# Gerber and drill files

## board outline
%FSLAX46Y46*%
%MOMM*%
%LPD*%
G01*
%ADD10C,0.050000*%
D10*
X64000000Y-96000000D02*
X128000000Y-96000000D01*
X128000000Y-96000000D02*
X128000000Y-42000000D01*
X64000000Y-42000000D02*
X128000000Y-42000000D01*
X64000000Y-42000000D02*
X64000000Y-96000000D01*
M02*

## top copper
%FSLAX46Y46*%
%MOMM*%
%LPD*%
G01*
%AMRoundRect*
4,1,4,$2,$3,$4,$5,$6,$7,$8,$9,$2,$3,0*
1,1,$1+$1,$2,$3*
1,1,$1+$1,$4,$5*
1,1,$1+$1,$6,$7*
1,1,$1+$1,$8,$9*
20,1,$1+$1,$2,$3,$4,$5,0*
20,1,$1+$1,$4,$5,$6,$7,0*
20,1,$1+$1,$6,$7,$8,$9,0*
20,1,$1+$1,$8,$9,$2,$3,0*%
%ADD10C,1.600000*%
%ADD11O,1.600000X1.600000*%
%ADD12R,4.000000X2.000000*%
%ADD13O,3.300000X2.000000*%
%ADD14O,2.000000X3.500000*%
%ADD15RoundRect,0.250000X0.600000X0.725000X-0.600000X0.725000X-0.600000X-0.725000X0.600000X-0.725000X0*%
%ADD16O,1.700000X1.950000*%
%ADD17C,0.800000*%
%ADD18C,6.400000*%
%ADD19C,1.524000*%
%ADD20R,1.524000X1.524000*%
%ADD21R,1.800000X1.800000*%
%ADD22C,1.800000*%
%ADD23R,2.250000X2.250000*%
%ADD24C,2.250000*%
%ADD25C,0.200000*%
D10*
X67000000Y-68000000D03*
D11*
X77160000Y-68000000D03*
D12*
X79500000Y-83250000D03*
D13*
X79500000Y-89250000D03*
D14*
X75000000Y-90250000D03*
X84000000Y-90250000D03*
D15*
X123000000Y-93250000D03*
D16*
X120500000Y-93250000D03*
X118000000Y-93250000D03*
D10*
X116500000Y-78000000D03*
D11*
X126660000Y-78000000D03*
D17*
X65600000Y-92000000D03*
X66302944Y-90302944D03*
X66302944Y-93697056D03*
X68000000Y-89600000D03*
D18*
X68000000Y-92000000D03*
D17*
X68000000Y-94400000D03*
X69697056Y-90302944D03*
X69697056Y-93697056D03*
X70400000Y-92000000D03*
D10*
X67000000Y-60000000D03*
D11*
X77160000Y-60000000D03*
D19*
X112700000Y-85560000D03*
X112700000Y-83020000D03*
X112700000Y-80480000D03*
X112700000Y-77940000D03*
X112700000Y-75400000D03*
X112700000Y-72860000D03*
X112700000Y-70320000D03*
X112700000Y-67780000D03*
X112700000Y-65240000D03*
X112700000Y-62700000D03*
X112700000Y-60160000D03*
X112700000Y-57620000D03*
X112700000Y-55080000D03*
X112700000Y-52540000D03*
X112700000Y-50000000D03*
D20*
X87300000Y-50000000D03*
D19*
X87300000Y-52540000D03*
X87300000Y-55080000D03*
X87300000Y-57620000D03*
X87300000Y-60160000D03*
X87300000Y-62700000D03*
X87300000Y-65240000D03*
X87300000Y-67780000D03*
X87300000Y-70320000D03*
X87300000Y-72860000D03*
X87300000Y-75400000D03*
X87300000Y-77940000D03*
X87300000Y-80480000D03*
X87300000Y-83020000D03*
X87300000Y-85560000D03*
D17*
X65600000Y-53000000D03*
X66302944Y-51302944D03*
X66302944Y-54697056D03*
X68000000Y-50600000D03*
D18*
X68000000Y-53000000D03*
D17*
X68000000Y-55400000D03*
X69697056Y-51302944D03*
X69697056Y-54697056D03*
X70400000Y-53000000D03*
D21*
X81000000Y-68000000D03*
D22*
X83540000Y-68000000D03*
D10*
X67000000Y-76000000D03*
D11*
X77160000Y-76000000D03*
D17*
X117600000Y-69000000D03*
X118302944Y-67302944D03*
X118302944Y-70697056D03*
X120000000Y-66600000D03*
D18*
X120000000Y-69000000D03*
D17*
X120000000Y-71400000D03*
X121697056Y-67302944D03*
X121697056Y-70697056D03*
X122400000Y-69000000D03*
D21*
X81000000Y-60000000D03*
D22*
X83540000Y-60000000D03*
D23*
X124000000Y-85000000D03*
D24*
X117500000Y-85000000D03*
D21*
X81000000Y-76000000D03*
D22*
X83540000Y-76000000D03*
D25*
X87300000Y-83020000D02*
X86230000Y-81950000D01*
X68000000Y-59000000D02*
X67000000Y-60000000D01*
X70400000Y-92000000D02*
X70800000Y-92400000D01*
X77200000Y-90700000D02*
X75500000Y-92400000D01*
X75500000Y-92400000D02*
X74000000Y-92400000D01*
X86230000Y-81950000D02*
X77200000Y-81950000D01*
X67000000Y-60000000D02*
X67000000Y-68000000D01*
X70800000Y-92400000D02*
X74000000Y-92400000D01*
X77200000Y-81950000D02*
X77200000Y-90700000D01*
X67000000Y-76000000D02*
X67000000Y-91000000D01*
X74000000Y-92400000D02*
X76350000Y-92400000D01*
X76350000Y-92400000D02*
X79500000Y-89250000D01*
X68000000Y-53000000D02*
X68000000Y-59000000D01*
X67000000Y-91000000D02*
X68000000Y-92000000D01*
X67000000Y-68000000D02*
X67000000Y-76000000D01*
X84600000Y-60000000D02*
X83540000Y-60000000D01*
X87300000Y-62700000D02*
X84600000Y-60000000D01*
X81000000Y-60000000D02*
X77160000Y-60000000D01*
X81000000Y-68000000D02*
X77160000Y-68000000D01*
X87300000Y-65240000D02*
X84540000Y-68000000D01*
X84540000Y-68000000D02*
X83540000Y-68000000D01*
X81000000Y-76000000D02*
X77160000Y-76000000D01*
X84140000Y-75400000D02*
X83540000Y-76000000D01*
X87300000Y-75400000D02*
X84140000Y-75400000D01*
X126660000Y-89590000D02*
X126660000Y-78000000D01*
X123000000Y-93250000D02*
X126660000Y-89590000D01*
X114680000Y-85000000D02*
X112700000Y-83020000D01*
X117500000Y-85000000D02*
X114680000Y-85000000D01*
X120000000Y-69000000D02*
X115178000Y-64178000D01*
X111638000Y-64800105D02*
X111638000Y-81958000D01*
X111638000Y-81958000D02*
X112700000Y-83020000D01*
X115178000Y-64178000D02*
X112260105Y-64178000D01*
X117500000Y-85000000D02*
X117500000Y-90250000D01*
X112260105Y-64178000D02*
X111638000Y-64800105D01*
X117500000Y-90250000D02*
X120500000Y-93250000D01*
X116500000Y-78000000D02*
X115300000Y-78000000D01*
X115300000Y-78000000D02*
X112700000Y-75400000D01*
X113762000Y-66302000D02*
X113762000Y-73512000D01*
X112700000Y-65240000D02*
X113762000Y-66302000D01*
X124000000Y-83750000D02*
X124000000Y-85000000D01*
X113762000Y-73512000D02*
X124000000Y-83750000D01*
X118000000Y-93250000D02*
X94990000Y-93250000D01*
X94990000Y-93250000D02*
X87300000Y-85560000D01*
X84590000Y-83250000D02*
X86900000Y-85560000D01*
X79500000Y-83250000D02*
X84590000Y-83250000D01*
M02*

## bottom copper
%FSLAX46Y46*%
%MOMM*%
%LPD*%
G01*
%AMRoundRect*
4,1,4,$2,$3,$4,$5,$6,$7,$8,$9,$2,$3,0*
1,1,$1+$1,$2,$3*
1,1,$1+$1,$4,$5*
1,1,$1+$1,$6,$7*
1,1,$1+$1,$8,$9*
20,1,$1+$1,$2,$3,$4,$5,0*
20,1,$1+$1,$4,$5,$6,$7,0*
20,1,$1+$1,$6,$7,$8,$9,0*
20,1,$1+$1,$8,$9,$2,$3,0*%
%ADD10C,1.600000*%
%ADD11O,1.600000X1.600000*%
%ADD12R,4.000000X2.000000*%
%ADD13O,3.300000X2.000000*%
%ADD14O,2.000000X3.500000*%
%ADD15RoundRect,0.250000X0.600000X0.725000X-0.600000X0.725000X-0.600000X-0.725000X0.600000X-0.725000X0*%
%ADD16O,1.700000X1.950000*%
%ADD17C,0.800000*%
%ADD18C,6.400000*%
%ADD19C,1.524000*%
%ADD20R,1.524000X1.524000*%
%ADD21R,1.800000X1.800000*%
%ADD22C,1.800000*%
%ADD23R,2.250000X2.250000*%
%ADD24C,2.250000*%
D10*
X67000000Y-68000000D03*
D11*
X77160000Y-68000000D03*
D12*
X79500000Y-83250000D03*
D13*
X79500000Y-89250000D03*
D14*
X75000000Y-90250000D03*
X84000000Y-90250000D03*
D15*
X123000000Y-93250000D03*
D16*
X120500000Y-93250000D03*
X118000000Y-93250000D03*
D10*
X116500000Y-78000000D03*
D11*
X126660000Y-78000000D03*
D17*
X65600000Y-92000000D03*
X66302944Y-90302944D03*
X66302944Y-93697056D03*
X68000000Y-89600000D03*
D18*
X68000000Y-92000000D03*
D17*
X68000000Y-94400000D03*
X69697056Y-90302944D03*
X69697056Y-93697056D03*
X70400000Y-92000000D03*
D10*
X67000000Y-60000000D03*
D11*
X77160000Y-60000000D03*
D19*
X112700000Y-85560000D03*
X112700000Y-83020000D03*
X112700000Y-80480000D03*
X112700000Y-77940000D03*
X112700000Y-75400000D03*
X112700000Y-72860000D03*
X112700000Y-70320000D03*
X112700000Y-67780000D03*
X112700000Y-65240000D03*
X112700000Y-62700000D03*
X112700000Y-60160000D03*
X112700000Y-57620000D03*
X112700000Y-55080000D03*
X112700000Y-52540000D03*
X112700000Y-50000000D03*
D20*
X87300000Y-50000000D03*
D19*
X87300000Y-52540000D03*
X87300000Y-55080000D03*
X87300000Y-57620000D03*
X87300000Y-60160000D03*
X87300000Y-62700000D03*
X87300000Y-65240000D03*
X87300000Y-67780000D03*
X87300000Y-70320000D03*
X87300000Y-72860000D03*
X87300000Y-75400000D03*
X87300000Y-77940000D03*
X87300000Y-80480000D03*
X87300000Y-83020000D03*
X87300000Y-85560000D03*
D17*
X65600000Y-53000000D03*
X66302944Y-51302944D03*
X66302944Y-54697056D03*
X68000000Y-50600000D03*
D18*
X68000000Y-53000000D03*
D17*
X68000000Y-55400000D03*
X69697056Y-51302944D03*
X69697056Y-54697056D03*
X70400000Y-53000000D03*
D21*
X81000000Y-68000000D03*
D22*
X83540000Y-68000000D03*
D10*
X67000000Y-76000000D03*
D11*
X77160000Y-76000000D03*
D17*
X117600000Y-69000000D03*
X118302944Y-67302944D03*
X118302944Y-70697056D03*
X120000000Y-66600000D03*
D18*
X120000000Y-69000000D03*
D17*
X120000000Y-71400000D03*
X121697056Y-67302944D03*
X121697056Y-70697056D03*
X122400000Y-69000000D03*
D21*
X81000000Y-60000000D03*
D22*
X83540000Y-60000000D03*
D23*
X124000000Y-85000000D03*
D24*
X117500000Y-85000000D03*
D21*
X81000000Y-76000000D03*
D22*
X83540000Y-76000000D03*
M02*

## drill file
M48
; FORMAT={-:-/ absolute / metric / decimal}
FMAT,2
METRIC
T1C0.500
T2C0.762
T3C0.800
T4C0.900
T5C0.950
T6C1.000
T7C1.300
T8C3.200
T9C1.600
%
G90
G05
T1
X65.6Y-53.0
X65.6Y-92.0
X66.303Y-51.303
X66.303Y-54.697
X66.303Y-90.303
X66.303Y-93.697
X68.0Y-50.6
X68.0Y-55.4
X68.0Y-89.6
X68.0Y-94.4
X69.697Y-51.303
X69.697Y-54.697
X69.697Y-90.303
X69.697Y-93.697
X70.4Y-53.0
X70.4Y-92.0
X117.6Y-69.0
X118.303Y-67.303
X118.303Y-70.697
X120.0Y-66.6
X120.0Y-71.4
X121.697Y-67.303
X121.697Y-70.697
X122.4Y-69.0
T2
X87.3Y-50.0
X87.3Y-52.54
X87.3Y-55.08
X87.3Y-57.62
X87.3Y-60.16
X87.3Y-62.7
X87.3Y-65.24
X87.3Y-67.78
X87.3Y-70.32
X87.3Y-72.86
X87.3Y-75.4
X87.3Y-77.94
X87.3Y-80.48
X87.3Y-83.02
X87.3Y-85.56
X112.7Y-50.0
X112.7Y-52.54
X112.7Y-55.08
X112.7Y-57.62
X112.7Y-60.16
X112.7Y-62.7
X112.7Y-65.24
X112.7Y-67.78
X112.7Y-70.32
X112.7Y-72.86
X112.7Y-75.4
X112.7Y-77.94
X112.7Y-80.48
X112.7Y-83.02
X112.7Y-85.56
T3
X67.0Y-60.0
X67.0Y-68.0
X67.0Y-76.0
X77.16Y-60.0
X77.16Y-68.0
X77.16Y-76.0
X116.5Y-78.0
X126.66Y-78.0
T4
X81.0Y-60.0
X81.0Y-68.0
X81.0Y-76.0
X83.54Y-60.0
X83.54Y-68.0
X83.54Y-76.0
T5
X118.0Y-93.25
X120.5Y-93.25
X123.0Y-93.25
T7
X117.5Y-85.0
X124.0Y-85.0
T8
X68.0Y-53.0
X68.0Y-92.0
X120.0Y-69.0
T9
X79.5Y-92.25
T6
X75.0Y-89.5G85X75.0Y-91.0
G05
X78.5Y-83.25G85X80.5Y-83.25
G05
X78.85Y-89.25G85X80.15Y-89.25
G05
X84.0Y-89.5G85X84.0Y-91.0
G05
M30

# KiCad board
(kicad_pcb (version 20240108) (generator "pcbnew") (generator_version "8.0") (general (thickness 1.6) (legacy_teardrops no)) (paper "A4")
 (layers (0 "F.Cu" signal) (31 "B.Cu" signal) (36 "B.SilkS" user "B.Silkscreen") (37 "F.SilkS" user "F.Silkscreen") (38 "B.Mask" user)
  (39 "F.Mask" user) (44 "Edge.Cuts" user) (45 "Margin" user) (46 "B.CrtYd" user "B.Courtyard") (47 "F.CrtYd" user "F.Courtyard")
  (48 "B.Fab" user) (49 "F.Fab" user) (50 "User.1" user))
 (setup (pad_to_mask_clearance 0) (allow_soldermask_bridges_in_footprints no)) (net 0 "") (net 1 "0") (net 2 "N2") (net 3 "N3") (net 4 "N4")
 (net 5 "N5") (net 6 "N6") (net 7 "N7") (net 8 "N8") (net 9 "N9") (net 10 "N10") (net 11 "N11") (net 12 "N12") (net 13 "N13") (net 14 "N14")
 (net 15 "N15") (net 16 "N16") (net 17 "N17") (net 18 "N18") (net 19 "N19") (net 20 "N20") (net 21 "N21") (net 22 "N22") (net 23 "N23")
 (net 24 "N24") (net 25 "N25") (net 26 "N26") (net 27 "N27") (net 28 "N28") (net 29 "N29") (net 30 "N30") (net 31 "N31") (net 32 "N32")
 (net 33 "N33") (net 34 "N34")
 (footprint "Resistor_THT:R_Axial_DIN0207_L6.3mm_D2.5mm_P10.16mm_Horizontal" (layer "F.Cu") (at 67 68)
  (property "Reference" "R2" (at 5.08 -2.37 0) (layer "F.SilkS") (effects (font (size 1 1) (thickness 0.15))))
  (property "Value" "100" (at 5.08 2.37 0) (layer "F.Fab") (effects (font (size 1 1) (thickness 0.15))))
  (pad "1" thru_hole circle (at 0 0) (size 1.6 1.6) (drill 0.8) (layers "*.Cu" "*.Mask") (remove_unused_layers no) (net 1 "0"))
  (pad "2" thru_hole oval (at 10.16 0) (size 1.6 1.6) (drill 0.8) (layers "*.Cu" "*.Mask") (remove_unused_layers no) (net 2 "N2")))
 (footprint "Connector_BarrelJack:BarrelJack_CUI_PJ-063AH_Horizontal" (layer "F.Cu") (at 79.5 83.25)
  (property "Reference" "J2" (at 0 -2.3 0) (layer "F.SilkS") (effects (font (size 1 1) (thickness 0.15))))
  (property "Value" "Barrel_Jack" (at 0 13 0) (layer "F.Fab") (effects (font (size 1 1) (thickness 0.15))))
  (pad "" np_thru_hole circle (at 0 9) (size 1.6 1.6) (drill 1.6) (layers "*.Cu" "*.Mask"))
  (pad "1" thru_hole rect (at 0 0) (size 4 2) (drill oval 3 1) (layers "*.Cu" "*.Mask") (remove_unused_layers no) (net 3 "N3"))
  (pad "2" thru_hole oval (at 0 6) (size 3.3 2) (drill oval 2.3 1) (layers "*.Cu" "*.Mask") (remove_unused_layers no) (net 1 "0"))
  (pad "MP" thru_hole oval (at -4.5 7) (size 2 3.5) (drill oval 1 2.5) (layers "*.Cu" "*.Mask") (remove_unused_layers no))
  (pad "MP" thru_hole oval (at 4.5 7) (size 2 3.5) (drill oval 1 2.5) (layers "*.Cu" "*.Mask") (remove_unused_layers no)))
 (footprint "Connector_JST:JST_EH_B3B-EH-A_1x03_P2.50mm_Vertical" (layer "F.Cu") (at 123 93.25 180)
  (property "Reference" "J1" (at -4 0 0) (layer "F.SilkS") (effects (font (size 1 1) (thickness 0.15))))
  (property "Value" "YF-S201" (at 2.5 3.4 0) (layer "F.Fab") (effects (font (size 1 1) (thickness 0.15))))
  (pad "1" thru_hole roundrect (at 0 0 180) (size 1.7 1.95) (drill 0.95) (layers "*.Cu" "*.Mask") (remove_unused_layers no)
   (roundrect_rratio 0.147059) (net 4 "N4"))
  (pad "2" thru_hole oval (at 2.5 0 180) (size 1.7 1.95) (drill 0.95) (layers "*.Cu" "*.Mask") (remove_unused_layers no) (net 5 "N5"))
  (pad "3" thru_hole oval (at 5 0 180) (size 1.7 1.95) (drill 0.95) (layers "*.Cu" "*.Mask") (remove_unused_layers no) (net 3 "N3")))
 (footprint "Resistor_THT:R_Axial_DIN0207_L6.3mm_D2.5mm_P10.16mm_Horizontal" (layer "F.Cu") (at 116.5 78)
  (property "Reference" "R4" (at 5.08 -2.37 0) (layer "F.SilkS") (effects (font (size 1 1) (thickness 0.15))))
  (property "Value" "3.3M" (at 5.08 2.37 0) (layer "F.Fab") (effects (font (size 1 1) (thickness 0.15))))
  (pad "1" thru_hole circle (at 0 0) (size 1.6 1.6) (drill 0.8) (layers "*.Cu" "*.Mask") (remove_unused_layers no) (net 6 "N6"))
  (pad "2" thru_hole oval (at 10.16 0) (size 1.6 1.6) (drill 0.8) (layers "*.Cu" "*.Mask") (remove_unused_layers no) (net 4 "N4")))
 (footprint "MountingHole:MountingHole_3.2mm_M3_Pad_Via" (layer "F.Cu") (at 68 92)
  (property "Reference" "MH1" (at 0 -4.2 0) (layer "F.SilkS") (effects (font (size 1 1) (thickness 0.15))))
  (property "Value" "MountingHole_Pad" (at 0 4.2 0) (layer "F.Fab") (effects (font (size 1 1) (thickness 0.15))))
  (pad "1" thru_hole circle (at -2.4 0) (size 0.8 0.8) (drill 0.5) (layers "*.Cu" "*.Mask") (remove_unused_layers no) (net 1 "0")
   (zone_connect 2))
  (pad "1" thru_hole circle (at -1.697056 -1.697056) (size 0.8 0.8) (drill 0.5) (layers "*.Cu" "*.Mask") (remove_unused_layers no)
   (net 1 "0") (zone_connect 2))
  (pad "1" thru_hole circle (at -1.697056 1.697056) (size 0.8 0.8) (drill 0.5) (layers "*.Cu" "*.Mask") (remove_unused_layers no)
   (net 1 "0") (zone_connect 2))
  (pad "1" thru_hole circle (at 0 -2.4) (size 0.8 0.8) (drill 0.5) (layers "*.Cu" "*.Mask") (remove_unused_layers no) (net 1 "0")
   (zone_connect 2))
  (pad "1" thru_hole circle (at 0 0) (size 6.4 6.4) (drill 3.2) (layers "*.Cu" "*.Mask") (remove_unused_layers no) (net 1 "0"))
  (pad "1" thru_hole circle (at 0 2.4) (size 0.8 0.8) (drill 0.5) (layers "*.Cu" "*.Mask") (remove_unused_layers no) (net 1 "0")
   (zone_connect 2))
  (pad "1" thru_hole circle (at 1.697056 -1.697056) (size 0.8 0.8) (drill 0.5) (layers "*.Cu" "*.Mask") (remove_unused_layers no)
   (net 1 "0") (zone_connect 2))
  (pad "1" thru_hole circle (at 1.697056 1.697056) (size 0.8 0.8) (drill 0.5) (layers "*.Cu" "*.Mask") (remove_unused_layers no) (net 1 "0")
   (zone_connect 2))
  (pad "1" thru_hole circle (at 2.4 0) (size 0.8 0.8) (drill 0.5) (layers "*.Cu" "*.Mask") (remove_unused_layers no) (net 1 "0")
   (zone_connect 2)))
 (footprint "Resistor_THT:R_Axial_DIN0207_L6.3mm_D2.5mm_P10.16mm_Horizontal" (layer "F.Cu") (at 67 60)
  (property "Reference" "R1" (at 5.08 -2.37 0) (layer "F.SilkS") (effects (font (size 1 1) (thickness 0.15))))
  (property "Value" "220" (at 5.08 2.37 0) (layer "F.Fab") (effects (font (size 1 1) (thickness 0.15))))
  (pad "1" thru_hole circle (at 0 0) (size 1.6 1.6) (drill 0.8) (layers "*.Cu" "*.Mask") (remove_unused_layers no) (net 1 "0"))
  (pad "2" thru_hole oval (at 10.16 0) (size 1.6 1.6) (drill 0.8) (layers "*.Cu" "*.Mask") (remove_unused_layers no) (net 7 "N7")))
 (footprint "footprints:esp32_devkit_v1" (layer "F.Cu") (at 100 50)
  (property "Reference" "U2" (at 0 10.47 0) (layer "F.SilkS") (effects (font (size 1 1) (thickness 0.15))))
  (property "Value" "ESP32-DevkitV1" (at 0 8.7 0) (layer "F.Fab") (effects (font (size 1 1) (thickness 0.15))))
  (pad "1" thru_hole circle (at 12.7 35.56) (size 1.524 1.524) (drill 0.762) (layers "*.Cu" "*.Mask") (remove_unused_layers no) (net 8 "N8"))
  (pad "2" thru_hole circle (at 12.7 33.02) (size 1.524 1.524) (drill 0.762) (layers "*.Cu" "*.Mask") (remove_unused_layers no) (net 5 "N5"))
  (pad "3" thru_hole circle (at 12.7 30.48) (size 1.524 1.524) (drill 0.762) (layers "*.Cu" "*.Mask") (remove_unused_layers no) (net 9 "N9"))
  (pad "4" thru_hole circle (at 12.7 27.94) (size 1.524 1.524) (drill 0.762) (layers "*.Cu" "*.Mask") (remove_unused_layers no)
   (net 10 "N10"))
  (pad "5" thru_hole circle (at 12.7 25.4) (size 1.524 1.524) (drill 0.762) (layers "*.Cu" "*.Mask") (remove_unused_layers no) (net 6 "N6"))
  (pad "6" thru_hole circle (at 12.7 22.86) (size 1.524 1.524) (drill 0.762) (layers "*.Cu" "*.Mask") (remove_unused_layers no)
   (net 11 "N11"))
  (pad "7" thru_hole circle (at 12.7 20.32) (size 1.524 1.524) (drill 0.762) (layers "*.Cu" "*.Mask") (remove_unused_layers no)
   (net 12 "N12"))
  (pad "8" thru_hole circle (at 12.7 17.78) (size 1.524 1.524) (drill 0.762) (layers "*.Cu" "*.Mask") (remove_unused_layers no)
   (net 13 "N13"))
  (pad "9" thru_hole circle (at 12.7 15.24) (size 1.524 1.524) (drill 0.762) (layers "*.Cu" "*.Mask") (remove_unused_layers no)
   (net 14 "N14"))
  (pad "10" thru_hole circle (at 12.7 12.7) (size 1.524 1.524) (drill 0.762) (layers "*.Cu" "*.Mask") (remove_unused_layers no)
   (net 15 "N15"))
  (pad "11" thru_hole circle (at 12.7 10.16) (size 1.524 1.524) (drill 0.762) (layers "*.Cu" "*.Mask") (remove_unused_layers no)
   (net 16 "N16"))
  (pad "12" thru_hole circle (at 12.7 7.62) (size 1.524 1.524) (drill 0.762) (layers "*.Cu" "*.Mask") (remove_unused_layers no)
   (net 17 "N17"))
  (pad "13" thru_hole circle (at 12.7 5.08) (size 1.524 1.524) (drill 0.762) (layers "*.Cu" "*.Mask") (remove_unused_layers no)
   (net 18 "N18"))
  (pad "14" thru_hole circle (at 12.7 2.54) (size 1.524 1.524) (drill 0.762) (layers "*.Cu" "*.Mask") (remove_unused_layers no)
   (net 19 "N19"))
  (pad "15" thru_hole circle (at 12.7 0) (size 1.524 1.524) (drill 0.762) (layers "*.Cu" "*.Mask") (remove_unused_layers no) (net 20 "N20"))
  (pad "16" thru_hole rect (at -12.7 0) (size 1.524 1.524) (drill 0.762) (layers "*.Cu" "*.Mask") (remove_unused_layers no) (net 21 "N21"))
  (pad "17" thru_hole circle (at -12.7 2.54) (size 1.524 1.524) (drill 0.762) (layers "*.Cu" "*.Mask") (remove_unused_layers no)
   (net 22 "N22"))
  (pad "18" thru_hole circle (at -12.7 5.08) (size 1.524 1.524) (drill 0.762) (layers "*.Cu" "*.Mask") (remove_unused_layers no)
   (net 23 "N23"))
  (pad "19" thru_hole circle (at -12.7 7.62) (size 1.524 1.524) (drill 0.762) (layers "*.Cu" "*.Mask") (remove_unused_layers no)
   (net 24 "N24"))
  (pad "20" thru_hole circle (at -12.7 10.16) (size 1.524 1.524) (drill 0.762) (layers "*.Cu" "*.Mask") (remove_unused_layers no)
   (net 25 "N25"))
  (pad "21" thru_hole circle (at -12.7 12.7) (size 1.524 1.524) (drill 0.762) (layers "*.Cu" "*.Mask") (remove_unused_layers no)
   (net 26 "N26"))
  (pad "22" thru_hole circle (at -12.7 15.24) (size 1.524 1.524) (drill 0.762) (layers "*.Cu" "*.Mask") (remove_unused_layers no)
   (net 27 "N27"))
  (pad "23" thru_hole circle (at -12.7 17.78) (size 1.524 1.524) (drill 0.762) (layers "*.Cu" "*.Mask") (remove_unused_layers no)
   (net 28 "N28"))
  (pad "24" thru_hole circle (at -12.7 20.32) (size 1.524 1.524) (drill 0.762) (layers "*.Cu" "*.Mask") (remove_unused_layers no)
   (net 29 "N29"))
  (pad "25" thru_hole circle (at -12.7 22.86) (size 1.524 1.524) (drill 0.762) (layers "*.Cu" "*.Mask") (remove_unused_layers no)
   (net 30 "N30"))
  (pad "26" thru_hole circle (at -12.7 25.4) (size 1.524 1.524) (drill 0.762) (layers "*.Cu" "*.Mask") (remove_unused_layers no)
   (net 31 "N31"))
  (pad "27" thru_hole circle (at -12.7 27.94) (size 1.524 1.524) (drill 0.762) (layers "*.Cu" "*.Mask") (remove_unused_layers no)
   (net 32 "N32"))
  (pad "28" thru_hole circle (at -12.7 30.48) (size 1.524 1.524) (drill 0.762) (layers "*.Cu" "*.Mask") (remove_unused_layers no)
   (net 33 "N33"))
  (pad "29" thru_hole circle (at -12.7 33.02) (size 1.524 1.524) (drill 0.762) (layers "*.Cu" "*.Mask") (remove_unused_layers no)
   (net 1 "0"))
  (pad "30" thru_hole circle (at -12.7 35.56) (size 1.524 1.524) (drill 0.762) (layers "*.Cu" "*.Mask") (remove_unused_layers no)
   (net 3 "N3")))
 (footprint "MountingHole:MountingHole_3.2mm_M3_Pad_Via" (layer "F.Cu") (at 68 53)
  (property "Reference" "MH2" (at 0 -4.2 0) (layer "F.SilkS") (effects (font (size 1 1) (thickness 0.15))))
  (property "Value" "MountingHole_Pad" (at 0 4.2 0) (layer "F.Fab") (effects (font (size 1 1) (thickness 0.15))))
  (pad "1" thru_hole circle (at -2.4 0) (size 0.8 0.8) (drill 0.5) (layers "*.Cu" "*.Mask") (remove_unused_layers no) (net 1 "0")
   (zone_connect 2))
  (pad "1" thru_hole circle (at -1.697056 -1.697056) (size 0.8 0.8) (drill 0.5) (layers "*.Cu" "*.Mask") (remove_unused_layers no)
   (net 1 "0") (zone_connect 2))
  (pad "1" thru_hole circle (at -1.697056 1.697056) (size 0.8 0.8) (drill 0.5) (layers "*.Cu" "*.Mask") (remove_unused_layers no)
   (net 1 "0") (zone_connect 2))
  (pad "1" thru_hole circle (at 0 -2.4) (size 0.8 0.8) (drill 0.5) (layers "*.Cu" "*.Mask") (remove_unused_layers no) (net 1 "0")
   (zone_connect 2))
  (pad "1" thru_hole circle (at 0 0) (size 6.4 6.4) (drill 3.2) (layers "*.Cu" "*.Mask") (remove_unused_layers no) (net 1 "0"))
  (pad "1" thru_hole circle (at 0 2.4) (size 0.8 0.8) (drill 0.5) (layers "*.Cu" "*.Mask") (remove_unused_layers no) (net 1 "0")
   (zone_connect 2))
  (pad "1" thru_hole circle (at 1.697056 -1.697056) (size 0.8 0.8) (drill 0.5) (layers "*.Cu" "*.Mask") (remove_unused_layers no)
   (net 1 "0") (zone_connect 2))
  (pad "1" thru_hole circle (at 1.697056 1.697056) (size 0.8 0.8) (drill 0.5) (layers "*.Cu" "*.Mask") (remove_unused_layers no) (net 1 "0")
   (zone_connect 2))
  (pad "1" thru_hole circle (at 2.4 0) (size 0.8 0.8) (drill 0.5) (layers "*.Cu" "*.Mask") (remove_unused_layers no) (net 1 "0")
   (zone_connect 2)))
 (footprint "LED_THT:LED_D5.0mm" (layer "F.Cu") (at 81 68)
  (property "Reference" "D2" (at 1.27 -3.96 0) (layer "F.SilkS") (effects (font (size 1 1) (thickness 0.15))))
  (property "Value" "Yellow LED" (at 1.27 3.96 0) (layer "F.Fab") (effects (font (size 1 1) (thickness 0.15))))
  (pad "1" thru_hole rect (at 0 0) (size 1.8 1.8) (drill 0.9) (layers "*.Cu" "*.Mask") (remove_unused_layers no) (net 2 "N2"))
  (pad "2" thru_hole circle (at 2.54 0) (size 1.8 1.8) (drill 0.9) (layers "*.Cu" "*.Mask") (remove_unused_layers no) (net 27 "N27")))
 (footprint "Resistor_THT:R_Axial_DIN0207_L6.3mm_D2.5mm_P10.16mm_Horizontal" (layer "F.Cu") (at 67 76)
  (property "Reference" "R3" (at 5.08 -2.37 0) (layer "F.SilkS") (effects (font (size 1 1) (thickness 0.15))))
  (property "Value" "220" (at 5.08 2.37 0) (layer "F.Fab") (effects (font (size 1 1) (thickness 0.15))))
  (pad "1" thru_hole circle (at 0 0) (size 1.6 1.6) (drill 0.8) (layers "*.Cu" "*.Mask") (remove_unused_layers no) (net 1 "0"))
  (pad "2" thru_hole oval (at 10.16 0) (size 1.6 1.6) (drill 0.8) (layers "*.Cu" "*.Mask") (remove_unused_layers no) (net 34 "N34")))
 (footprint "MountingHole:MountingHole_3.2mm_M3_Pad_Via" (layer "F.Cu") (at 120 69)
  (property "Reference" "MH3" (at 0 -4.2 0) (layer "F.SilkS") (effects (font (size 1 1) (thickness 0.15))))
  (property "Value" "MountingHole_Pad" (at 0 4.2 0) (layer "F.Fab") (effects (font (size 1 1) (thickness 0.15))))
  (pad "1" thru_hole circle (at -2.4 0) (size 0.8 0.8) (drill 0.5) (layers "*.Cu" "*.Mask") (remove_unused_layers no) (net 5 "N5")
   (zone_connect 2))
  (pad "1" thru_hole circle (at -1.697056 -1.697056) (size 0.8 0.8) (drill 0.5) (layers "*.Cu" "*.Mask") (remove_unused_layers no)
   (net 5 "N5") (zone_connect 2))
  (pad "1" thru_hole circle (at -1.697056 1.697056) (size 0.8 0.8) (drill 0.5) (layers "*.Cu" "*.Mask") (remove_unused_layers no)
   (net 5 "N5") (zone_connect 2))
  (pad "1" thru_hole circle (at 0 -2.4) (size 0.8 0.8) (drill 0.5) (layers "*.Cu" "*.Mask") (remove_unused_layers no) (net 5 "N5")
   (zone_connect 2))
  (pad "1" thru_hole circle (at 0 0) (size 6.4 6.4) (drill 3.2) (layers "*.Cu" "*.Mask") (remove_unused_layers no) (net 5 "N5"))
  (pad "1" thru_hole circle (at 0 2.4) (size 0.8 0.8) (drill 0.5) (layers "*.Cu" "*.Mask") (remove_unused_layers no) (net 5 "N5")
   (zone_connect 2))
  (pad "1" thru_hole circle (at 1.697056 -1.697056) (size 0.8 0.8) (drill 0.5) (layers "*.Cu" "*.Mask") (remove_unused_layers no)
   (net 5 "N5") (zone_connect 2))
  (pad "1" thru_hole circle (at 1.697056 1.697056) (size 0.8 0.8) (drill 0.5) (layers "*.Cu" "*.Mask") (remove_unused_layers no)
   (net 5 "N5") (zone_connect 2))
  (pad "1" thru_hole circle (at 2.4 0) (size 0.8 0.8) (drill 0.5) (layers "*.Cu" "*.Mask") (remove_unused_layers no) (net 5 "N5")
   (zone_connect 2)))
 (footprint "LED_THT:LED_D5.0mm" (layer "F.Cu") (at 81 60)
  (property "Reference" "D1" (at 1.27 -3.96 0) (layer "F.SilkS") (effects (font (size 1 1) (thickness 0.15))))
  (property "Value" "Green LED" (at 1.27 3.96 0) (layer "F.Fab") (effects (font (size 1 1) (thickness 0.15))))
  (pad "1" thru_hole rect (at 0 0) (size 1.8 1.8) (drill 0.9) (layers "*.Cu" "*.Mask") (remove_unused_layers no) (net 7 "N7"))
  (pad "2" thru_hole circle (at 2.54 0) (size 1.8 1.8) (drill 0.9) (layers "*.Cu" "*.Mask") (remove_unused_layers no) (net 26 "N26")))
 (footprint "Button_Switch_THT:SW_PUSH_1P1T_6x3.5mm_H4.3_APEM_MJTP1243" (layer "F.Cu") (at 124 85 180)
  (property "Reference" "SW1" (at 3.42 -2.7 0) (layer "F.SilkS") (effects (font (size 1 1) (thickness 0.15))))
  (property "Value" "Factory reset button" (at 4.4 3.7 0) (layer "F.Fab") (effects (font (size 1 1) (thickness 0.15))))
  (pad "1" thru_hole rect (at 0 0 270) (size 2.25 2.25) (drill 1.3) (layers "*.Cu" "*.Mask") (remove_unused_layers no) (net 14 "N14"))
  (pad "2" thru_hole circle (at 6.5 0 270) (size 2.25 2.25) (drill 1.3) (layers "*.Cu" "*.Mask") (remove_unused_layers no) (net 5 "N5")))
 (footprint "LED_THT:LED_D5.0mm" (layer "F.Cu") (at 81 76)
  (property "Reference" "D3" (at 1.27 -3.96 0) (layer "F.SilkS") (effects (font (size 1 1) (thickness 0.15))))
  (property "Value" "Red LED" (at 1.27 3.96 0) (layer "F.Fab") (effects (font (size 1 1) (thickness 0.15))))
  (pad "1" thru_hole rect (at 0 0) (size 1.8 1.8) (drill 0.9) (layers "*.Cu" "*.Mask") (remove_unused_layers no) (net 34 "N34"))
  (pad "2" thru_hole circle (at 2.54 0) (size 1.8 1.8) (drill 0.9) (layers "*.Cu" "*.Mask") (remove_unused_layers no) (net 31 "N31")))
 (gr_line (start 64 96) (end 128 96) (stroke (width 0.05) (type default)) (layer "Edge.Cuts"))
 (gr_line (start 128 96) (end 128 42) (stroke (width 0.05) (type default)) (layer "Edge.Cuts"))
 (gr_line (start 64 42) (end 128 42) (stroke (width 0.05) (type default)) (layer "Edge.Cuts"))
 (gr_line (start 64 42) (end 64 96) (stroke (width 0.05) (type default)) (layer "Edge.Cuts"))
 (segment (start 87.3 83.02) (end 86.23 81.95) (width 0.2) (layer "F.Cu") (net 1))
 (segment (start 68 59) (end 67 60) (width 0.2) (layer "F.Cu") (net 1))
 (segment (start 70.4 92) (end 70.8 92.4) (width 0.2) (layer "F.Cu") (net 1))
 (segment (start 77.2 90.7) (end 75.5 92.4) (width 0.2) (layer "F.Cu") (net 1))
 (segment (start 75.5 92.4) (end 74 92.4) (width 0.2) (layer "F.Cu") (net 1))
 (segment (start 86.23 81.95) (end 77.2 81.95) (width 0.2) (layer "F.Cu") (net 1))
 (segment (start 67 60) (end 67 68) (width 0.2) (layer "F.Cu") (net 1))
 (segment (start 70.8 92.4) (end 74 92.4) (width 0.2) (layer "F.Cu") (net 1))
 (segment (start 77.2 81.95) (end 77.2 90.7) (width 0.2) (layer "F.Cu") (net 1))
 (segment (start 67 76) (end 67 91) (width 0.2) (layer "F.Cu") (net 1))
 (segment (start 74 92.4) (end 76.35 92.4) (width 0.2) (layer "F.Cu") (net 1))
 (segment (start 76.35 92.4) (end 79.5 89.25) (width 0.2) (layer "F.Cu") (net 1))
 (segment (start 68 53) (end 68 59) (width 0.2) (layer "F.Cu") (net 1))
 (segment (start 67 91) (end 68 92) (width 0.2) (layer "F.Cu") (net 1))
 (segment (start 67 68) (end 67 76) (width 0.2) (layer "F.Cu") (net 1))
 (segment (start 84.6 60) (end 83.54 60) (width 0.2) (layer "F.Cu") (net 26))
 (segment (start 87.3 62.7) (end 84.6 60) (width 0.2) (layer "F.Cu") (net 26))
 (segment (start 81 60) (end 77.16 60) (width 0.2) (layer "F.Cu") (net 7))
 (segment (start 81 68) (end 77.16 68) (width 0.2) (layer "F.Cu") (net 2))
 (segment (start 87.3 65.24) (end 84.54 68) (width 0.2) (layer "F.Cu") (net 27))
 (segment (start 84.54 68) (end 83.54 68) (width 0.2) (layer "F.Cu") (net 27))
 (segment (start 81 76) (end 77.16 76) (width 0.2) (layer "F.Cu") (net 34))
 (segment (start 84.14 75.4) (end 83.54 76) (width 0.2) (layer "F.Cu") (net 31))
 (segment (start 87.3 75.4) (end 84.14 75.4) (width 0.2) (layer "F.Cu") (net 31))
 (segment (start 126.66 89.59) (end 126.66 78) (width 0.2) (layer "F.Cu") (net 4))
 (segment (start 123 93.25) (end 126.66 89.59) (width 0.2) (layer "F.Cu") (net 4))
 (segment (start 114.68 85) (end 112.7 83.02) (width 0.2) (layer "F.Cu") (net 5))
 (segment (start 117.5 85) (end 114.68 85) (width 0.2) (layer "F.Cu") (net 5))
 (segment (start 120 69) (end 115.178 64.178) (width 0.2) (layer "F.Cu") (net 5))
 (segment (start 111.638 64.800105) (end 111.638 81.958) (width 0.2) (layer "F.Cu") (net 5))
 (segment (start 111.638 81.958) (end 112.7 83.02) (width 0.2) (layer "F.Cu") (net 5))
 (segment (start 115.178 64.178) (end 112.260105 64.178) (width 0.2) (layer "F.Cu") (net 5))
 (segment (start 117.5 85) (end 117.5 90.25) (width 0.2) (layer "F.Cu") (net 5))
 (segment (start 112.260105 64.178) (end 111.638 64.800105) (width 0.2) (layer "F.Cu") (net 5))
 (segment (start 117.5 90.25) (end 120.5 93.25) (width 0.2) (layer "F.Cu") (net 5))
 (segment (start 116.5 78) (end 115.3 78) (width 0.2) (layer "F.Cu") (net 6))
 (segment (start 115.3 78) (end 112.7 75.4) (width 0.2) (layer "F.Cu") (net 6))
 (segment (start 113.762 66.302) (end 113.762 73.512) (width 0.2) (layer "F.Cu") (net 14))
 (segment (start 112.7 65.24) (end 113.762 66.302) (width 0.2) (layer "F.Cu") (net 14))
 (segment (start 124 83.75) (end 124 85) (width 0.2) (layer "F.Cu") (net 14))
 (segment (start 113.762 73.512) (end 124 83.75) (width 0.2) (layer "F.Cu") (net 14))
 (segment (start 118 93.25) (end 94.99 93.25) (width 0.2) (layer "F.Cu") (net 3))
 (segment (start 94.99 93.25) (end 87.3 85.56) (width 0.2) (layer "F.Cu") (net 3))
 (segment (start 84.59 83.25) (end 86.9 85.56) (width 0.2) (layer "F.Cu") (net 3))
 (segment (start 79.5 83.25) (end 84.59 83.25) (width 0.2) (layer "F.Cu") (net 3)))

